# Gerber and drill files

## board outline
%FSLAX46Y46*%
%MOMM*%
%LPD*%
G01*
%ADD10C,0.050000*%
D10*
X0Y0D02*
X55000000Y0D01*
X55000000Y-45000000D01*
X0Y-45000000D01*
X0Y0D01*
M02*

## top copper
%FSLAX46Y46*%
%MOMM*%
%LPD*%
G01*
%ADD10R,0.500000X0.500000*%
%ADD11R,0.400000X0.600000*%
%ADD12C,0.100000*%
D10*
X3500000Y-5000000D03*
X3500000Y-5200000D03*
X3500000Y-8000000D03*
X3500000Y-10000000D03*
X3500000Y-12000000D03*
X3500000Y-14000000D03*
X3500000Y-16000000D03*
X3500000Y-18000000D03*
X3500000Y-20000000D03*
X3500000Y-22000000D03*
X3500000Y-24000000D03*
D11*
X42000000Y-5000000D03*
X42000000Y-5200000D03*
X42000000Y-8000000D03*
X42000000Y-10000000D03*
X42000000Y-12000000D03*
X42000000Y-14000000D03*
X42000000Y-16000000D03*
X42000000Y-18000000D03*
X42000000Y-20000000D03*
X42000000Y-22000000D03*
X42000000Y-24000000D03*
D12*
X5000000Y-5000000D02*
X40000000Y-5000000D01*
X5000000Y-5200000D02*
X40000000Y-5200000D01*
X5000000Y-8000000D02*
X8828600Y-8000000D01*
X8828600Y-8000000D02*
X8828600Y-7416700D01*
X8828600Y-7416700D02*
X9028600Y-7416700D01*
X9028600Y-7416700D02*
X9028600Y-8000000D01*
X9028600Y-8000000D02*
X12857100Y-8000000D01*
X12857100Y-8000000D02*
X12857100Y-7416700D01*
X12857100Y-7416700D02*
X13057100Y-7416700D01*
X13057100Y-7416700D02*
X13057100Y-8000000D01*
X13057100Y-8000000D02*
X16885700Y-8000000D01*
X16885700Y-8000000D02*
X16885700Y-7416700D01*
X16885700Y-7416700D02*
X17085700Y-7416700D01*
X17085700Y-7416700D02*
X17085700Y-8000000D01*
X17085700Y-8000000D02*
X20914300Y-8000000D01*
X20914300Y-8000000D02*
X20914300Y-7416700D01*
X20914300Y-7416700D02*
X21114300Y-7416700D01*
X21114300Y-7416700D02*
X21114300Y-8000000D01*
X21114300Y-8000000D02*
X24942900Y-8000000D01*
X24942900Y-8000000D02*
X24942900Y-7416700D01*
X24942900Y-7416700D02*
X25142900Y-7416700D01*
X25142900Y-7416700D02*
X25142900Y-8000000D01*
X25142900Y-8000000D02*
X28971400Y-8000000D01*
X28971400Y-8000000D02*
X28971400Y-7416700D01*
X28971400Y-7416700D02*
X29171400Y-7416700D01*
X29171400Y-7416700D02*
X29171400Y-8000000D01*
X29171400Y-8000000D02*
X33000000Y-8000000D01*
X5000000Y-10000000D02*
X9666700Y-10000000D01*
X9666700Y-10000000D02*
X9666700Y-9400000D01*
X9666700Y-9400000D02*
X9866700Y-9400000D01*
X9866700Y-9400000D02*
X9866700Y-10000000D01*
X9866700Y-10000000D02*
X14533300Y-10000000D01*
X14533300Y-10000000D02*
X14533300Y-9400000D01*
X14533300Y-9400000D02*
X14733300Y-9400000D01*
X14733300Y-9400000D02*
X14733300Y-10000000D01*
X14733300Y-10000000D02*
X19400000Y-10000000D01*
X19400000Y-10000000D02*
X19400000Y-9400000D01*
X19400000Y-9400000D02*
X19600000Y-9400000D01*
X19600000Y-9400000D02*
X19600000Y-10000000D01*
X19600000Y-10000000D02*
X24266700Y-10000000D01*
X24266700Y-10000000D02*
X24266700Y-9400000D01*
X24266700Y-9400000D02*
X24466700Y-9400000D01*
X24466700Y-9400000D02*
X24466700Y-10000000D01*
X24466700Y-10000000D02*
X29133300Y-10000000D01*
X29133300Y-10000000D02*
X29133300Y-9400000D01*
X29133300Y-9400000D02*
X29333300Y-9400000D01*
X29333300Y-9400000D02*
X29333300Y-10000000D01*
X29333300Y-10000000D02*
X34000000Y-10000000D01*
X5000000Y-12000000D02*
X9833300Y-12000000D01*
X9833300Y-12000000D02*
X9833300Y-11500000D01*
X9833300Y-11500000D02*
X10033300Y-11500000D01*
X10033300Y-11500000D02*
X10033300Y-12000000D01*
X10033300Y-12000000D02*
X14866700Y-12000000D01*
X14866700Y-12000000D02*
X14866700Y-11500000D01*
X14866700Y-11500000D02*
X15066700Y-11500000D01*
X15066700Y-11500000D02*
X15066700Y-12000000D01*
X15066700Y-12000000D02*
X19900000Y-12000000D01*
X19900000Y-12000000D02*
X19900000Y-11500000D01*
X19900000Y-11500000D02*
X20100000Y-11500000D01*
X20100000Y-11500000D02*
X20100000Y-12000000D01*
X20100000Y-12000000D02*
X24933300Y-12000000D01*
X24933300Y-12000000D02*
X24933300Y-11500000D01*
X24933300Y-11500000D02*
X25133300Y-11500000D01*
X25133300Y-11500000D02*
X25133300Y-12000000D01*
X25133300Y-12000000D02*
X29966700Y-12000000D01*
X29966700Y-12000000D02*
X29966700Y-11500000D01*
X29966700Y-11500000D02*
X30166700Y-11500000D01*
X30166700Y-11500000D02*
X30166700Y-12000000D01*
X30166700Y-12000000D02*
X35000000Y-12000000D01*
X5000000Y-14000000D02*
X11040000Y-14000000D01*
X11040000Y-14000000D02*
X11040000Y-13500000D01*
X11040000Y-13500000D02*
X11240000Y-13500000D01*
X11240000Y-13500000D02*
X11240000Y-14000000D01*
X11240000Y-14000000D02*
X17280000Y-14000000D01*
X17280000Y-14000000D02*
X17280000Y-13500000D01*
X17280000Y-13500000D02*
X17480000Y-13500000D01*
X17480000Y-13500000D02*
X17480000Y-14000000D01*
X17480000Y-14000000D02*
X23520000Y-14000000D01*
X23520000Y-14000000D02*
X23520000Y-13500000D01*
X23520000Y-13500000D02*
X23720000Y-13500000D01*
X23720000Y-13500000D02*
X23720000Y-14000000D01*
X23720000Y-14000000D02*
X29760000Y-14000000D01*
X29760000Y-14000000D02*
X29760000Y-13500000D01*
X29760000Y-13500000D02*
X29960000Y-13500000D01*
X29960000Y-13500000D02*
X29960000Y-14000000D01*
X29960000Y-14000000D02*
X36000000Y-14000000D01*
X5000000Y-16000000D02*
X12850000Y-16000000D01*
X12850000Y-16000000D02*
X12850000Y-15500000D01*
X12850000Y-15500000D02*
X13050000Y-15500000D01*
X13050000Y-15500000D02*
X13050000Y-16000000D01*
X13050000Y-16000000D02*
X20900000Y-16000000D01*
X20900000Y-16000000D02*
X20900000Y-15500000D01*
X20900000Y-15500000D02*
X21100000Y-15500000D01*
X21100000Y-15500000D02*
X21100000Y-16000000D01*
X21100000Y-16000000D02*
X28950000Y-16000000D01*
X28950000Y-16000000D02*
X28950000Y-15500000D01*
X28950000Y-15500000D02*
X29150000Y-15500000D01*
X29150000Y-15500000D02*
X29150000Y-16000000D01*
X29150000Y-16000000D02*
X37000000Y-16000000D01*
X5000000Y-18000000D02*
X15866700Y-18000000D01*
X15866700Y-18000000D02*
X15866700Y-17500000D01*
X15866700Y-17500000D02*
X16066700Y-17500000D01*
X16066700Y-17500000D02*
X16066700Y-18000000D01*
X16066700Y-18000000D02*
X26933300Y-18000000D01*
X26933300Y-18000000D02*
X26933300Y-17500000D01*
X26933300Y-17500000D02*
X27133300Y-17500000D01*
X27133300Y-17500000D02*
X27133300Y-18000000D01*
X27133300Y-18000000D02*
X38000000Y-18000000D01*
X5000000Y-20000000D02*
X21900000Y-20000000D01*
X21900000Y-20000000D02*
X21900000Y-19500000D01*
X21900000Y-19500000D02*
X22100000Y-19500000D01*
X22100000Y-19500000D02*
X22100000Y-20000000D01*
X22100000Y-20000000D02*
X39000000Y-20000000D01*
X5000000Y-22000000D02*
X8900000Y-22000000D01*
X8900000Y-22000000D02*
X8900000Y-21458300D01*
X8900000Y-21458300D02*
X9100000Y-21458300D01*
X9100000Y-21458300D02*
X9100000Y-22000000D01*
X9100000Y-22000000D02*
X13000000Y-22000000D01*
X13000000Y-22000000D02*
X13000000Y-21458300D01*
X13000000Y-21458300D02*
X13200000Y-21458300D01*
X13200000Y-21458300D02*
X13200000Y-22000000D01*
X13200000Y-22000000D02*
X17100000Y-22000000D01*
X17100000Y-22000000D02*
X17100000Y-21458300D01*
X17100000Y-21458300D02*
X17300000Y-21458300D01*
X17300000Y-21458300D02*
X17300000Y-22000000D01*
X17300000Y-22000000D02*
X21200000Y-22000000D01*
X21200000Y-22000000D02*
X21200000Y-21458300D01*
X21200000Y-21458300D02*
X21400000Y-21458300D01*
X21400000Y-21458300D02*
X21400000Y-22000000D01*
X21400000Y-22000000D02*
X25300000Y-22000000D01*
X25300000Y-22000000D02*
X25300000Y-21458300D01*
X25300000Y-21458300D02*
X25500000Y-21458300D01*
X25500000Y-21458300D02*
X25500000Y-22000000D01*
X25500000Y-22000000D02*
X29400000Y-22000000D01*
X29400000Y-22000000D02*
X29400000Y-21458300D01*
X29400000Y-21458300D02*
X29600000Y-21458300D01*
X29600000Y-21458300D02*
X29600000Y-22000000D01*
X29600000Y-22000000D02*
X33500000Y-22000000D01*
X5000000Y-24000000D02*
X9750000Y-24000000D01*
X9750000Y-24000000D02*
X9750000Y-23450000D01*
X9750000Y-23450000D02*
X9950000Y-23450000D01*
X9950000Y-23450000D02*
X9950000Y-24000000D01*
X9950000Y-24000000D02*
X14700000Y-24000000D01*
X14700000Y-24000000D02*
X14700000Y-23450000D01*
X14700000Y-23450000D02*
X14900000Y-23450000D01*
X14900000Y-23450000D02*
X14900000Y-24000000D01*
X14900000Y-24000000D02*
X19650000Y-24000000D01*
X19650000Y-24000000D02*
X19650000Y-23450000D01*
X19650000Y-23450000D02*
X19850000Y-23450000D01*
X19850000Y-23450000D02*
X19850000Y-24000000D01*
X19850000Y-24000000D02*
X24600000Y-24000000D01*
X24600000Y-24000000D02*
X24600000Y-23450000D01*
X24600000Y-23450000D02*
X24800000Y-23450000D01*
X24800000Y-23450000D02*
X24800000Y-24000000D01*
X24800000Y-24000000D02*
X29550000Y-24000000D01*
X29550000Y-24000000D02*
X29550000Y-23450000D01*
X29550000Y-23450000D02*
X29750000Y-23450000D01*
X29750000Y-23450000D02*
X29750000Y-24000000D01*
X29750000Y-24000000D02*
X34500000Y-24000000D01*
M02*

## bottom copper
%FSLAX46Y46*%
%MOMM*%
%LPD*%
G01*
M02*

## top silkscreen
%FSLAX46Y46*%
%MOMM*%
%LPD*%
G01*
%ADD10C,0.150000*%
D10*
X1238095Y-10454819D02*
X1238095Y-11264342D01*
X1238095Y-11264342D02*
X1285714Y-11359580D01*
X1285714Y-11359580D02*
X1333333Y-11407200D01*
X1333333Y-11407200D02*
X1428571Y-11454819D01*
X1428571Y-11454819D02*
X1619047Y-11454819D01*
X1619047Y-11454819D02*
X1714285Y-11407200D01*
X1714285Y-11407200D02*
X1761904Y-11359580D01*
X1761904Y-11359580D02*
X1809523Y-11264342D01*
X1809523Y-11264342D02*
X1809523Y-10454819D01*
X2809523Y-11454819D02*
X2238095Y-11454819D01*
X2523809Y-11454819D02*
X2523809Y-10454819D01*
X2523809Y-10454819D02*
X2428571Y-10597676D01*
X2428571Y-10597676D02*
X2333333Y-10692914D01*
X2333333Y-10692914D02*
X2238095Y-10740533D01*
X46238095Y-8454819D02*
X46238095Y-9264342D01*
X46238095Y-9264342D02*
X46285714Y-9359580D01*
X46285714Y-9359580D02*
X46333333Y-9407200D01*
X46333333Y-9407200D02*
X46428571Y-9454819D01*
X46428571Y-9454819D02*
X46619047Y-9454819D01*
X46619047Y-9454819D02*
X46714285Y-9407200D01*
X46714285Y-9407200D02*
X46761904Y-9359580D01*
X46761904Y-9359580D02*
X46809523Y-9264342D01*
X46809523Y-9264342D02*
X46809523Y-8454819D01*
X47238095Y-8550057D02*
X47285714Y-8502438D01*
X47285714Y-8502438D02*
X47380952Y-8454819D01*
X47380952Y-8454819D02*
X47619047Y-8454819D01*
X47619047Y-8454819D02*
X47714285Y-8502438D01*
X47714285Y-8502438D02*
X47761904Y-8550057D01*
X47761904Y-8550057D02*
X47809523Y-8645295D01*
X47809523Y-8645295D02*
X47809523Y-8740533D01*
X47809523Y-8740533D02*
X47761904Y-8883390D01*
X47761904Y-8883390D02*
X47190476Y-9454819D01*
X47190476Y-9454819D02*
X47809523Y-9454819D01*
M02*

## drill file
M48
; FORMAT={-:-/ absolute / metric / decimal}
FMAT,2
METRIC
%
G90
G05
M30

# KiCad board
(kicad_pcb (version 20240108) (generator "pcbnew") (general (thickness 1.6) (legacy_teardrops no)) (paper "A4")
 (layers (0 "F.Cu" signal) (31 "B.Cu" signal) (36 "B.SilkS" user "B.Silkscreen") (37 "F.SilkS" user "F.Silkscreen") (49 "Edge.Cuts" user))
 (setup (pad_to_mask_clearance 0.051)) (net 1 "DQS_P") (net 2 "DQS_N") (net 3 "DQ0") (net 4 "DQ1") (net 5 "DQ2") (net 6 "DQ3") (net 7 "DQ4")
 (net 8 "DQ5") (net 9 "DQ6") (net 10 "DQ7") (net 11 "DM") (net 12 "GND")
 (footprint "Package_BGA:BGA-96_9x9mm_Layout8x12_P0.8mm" (layer "F.Cu") (at 2 18)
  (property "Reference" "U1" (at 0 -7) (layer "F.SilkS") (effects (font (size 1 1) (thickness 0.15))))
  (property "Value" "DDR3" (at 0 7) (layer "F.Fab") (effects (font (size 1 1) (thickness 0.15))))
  (pad "A1" smd rect (at 1.5 -13) (size 0.5 0.5) (layers "F.Cu" "F.Paste" "F.Mask") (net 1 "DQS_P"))
  (pad "A2" smd rect (at 1.5 -12.8) (size 0.5 0.5) (layers "F.Cu" "F.Paste" "F.Mask") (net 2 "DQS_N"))
  (pad "B1" smd rect (at 1.5 -10) (size 0.5 0.5) (layers "F.Cu" "F.Paste" "F.Mask") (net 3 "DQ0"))
  (pad "B2" smd rect (at 1.5 -8) (size 0.5 0.5) (layers "F.Cu" "F.Paste" "F.Mask") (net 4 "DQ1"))
  (pad "B3" smd rect (at 1.5 -6) (size 0.5 0.5) (layers "F.Cu" "F.Paste" "F.Mask") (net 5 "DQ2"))
  (pad "B4" smd rect (at 1.5 -4) (size 0.5 0.5) (layers "F.Cu" "F.Paste" "F.Mask") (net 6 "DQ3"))
  (pad "B5" smd rect (at 1.5 -2) (size 0.5 0.5) (layers "F.Cu" "F.Paste" "F.Mask") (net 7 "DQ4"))
  (pad "B6" smd rect (at 1.5 0) (size 0.5 0.5) (layers "F.Cu" "F.Paste" "F.Mask") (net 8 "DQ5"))
  (pad "B7" smd rect (at 1.5 2) (size 0.5 0.5) (layers "F.Cu" "F.Paste" "F.Mask") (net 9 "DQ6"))
  (pad "B8" smd rect (at 1.5 4) (size 0.5 0.5) (layers "F.Cu" "F.Paste" "F.Mask") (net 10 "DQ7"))
  (pad "B9" smd rect (at 1.5 6) (size 0.5 0.5) (layers "F.Cu" "F.Paste" "F.Mask") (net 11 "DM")))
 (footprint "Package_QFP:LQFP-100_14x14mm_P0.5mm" (layer "F.Cu") (at 47 18)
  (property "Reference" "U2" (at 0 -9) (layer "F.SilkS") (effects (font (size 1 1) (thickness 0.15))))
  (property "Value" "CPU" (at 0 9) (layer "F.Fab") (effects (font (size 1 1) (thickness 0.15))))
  (pad "1" smd rect (at -5 -13) (size 0.4 0.6) (layers "F.Cu" "F.Paste" "F.Mask") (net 1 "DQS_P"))
  (pad "2" smd rect (at -5 -12.8) (size 0.4 0.6) (layers "F.Cu" "F.Paste" "F.Mask") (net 2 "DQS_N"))
  (pad "3" smd rect (at -5 -10) (size 0.4 0.6) (layers "F.Cu" "F.Paste" "F.Mask") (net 3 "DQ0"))
  (pad "4" smd rect (at -5 -8) (size 0.4 0.6) (layers "F.Cu" "F.Paste" "F.Mask") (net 4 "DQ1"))
  (pad "5" smd rect (at -5 -6) (size 0.4 0.6) (layers "F.Cu" "F.Paste" "F.Mask") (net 5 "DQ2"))
  (pad "6" smd rect (at -5 -4) (size 0.4 0.6) (layers "F.Cu" "F.Paste" "F.Mask") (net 6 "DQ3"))
  (pad "7" smd rect (at -5 -2) (size 0.4 0.6) (layers "F.Cu" "F.Paste" "F.Mask") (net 7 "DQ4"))
  (pad "8" smd rect (at -5 0) (size 0.4 0.6) (layers "F.Cu" "F.Paste" "F.Mask") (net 8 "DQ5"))
  (pad "9" smd rect (at -5 2) (size 0.4 0.6) (layers "F.Cu" "F.Paste" "F.Mask") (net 9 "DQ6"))
  (pad "10" smd rect (at -5 4) (size 0.4 0.6) (layers "F.Cu" "F.Paste" "F.Mask") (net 10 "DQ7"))
  (pad "11" smd rect (at -5 6) (size 0.4 0.6) (layers "F.Cu" "F.Paste" "F.Mask") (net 11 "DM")))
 (segment (start 5 5) (end 40 5) (width 0.1) (layer "F.Cu") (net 1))
 (segment (start 5 5.2) (end 40 5.2) (width 0.1) (layer "F.Cu") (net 2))
 (segment (start 5.0000 8.0) (end 8.8286 8.0) (width 0.1) (layer "F.Cu") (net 3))
 (segment (start 8.8286 8.0) (end 8.8286 7.4167) (width 0.1) (layer "F.Cu") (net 3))
 (segment (start 8.8286 7.4167) (end 9.0286 7.4167) (width 0.1) (layer "F.Cu") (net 3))
 (segment (start 9.0286 7.4167) (end 9.0286 8.0) (width 0.1) (layer "F.Cu") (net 3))
 (segment (start 9.0286 8.0) (end 12.8571 8.0) (width 0.1) (layer "F.Cu") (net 3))
 (segment (start 12.8571 8.0) (end 12.8571 7.4167) (width 0.1) (layer "F.Cu") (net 3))
 (segment (start 12.8571 7.4167) (end 13.0571 7.4167) (width 0.1) (layer "F.Cu") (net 3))
 (segment (start 13.0571 7.4167) (end 13.0571 8.0) (width 0.1) (layer "F.Cu") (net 3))
 (segment (start 13.0571 8.0) (end 16.8857 8.0) (width 0.1) (layer "F.Cu") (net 3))
 (segment (start 16.8857 8.0) (end 16.8857 7.4167) (width 0.1) (layer "F.Cu") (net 3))
 (segment (start 16.8857 7.4167) (end 17.0857 7.4167) (width 0.1) (layer "F.Cu") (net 3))
 (segment (start 17.0857 7.4167) (end 17.0857 8.0) (width 0.1) (layer "F.Cu") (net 3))
 (segment (start 17.0857 8.0) (end 20.9143 8.0) (width 0.1) (layer "F.Cu") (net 3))
 (segment (start 20.9143 8.0) (end 20.9143 7.4167) (width 0.1) (layer "F.Cu") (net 3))
 (segment (start 20.9143 7.4167) (end 21.1143 7.4167) (width 0.1) (layer "F.Cu") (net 3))
 (segment (start 21.1143 7.4167) (end 21.1143 8.0) (width 0.1) (layer "F.Cu") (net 3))
 (segment (start 21.1143 8.0) (end 24.9429 8.0) (width 0.1) (layer "F.Cu") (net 3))
 (segment (start 24.9429 8.0) (end 24.9429 7.4167) (width 0.1) (layer "F.Cu") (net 3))
 (segment (start 24.9429 7.4167) (end 25.1429 7.4167) (width 0.1) (layer "F.Cu") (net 3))
 (segment (start 25.1429 7.4167) (end 25.1429 8.0) (width 0.1) (layer "F.Cu") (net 3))
 (segment (start 25.1429 8.0) (end 28.9714 8.0) (width 0.1) (layer "F.Cu") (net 3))
 (segment (start 28.9714 8.0) (end 28.9714 7.4167) (width 0.1) (layer "F.Cu") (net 3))
 (segment (start 28.9714 7.4167) (end 29.1714 7.4167) (width 0.1) (layer "F.Cu") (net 3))
 (segment (start 29.1714 7.4167) (end 29.1714 8.0) (width 0.1) (layer "F.Cu") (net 3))
 (segment (start 29.1714 8.0) (end 33.0 8.0) (width 0.1) (layer "F.Cu") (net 3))
 (segment (start 5.0000 10.0) (end 9.6667 10.0) (width 0.1) (layer "F.Cu") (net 4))
 (segment (start 9.6667 10.0) (end 9.6667 9.4000) (width 0.1) (layer "F.Cu") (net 4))
 (segment (start 9.6667 9.4000) (end 9.8667 9.4000) (width 0.1) (layer "F.Cu") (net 4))
 (segment (start 9.8667 9.4000) (end 9.8667 10.0) (width 0.1) (layer "F.Cu") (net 4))
 (segment (start 9.8667 10.0) (end 14.5333 10.0) (width 0.1) (layer "F.Cu") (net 4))
 (segment (start 14.5333 10.0) (end 14.5333 9.4000) (width 0.1) (layer "F.Cu") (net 4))
 (segment (start 14.5333 9.4000) (end 14.7333 9.4000) (width 0.1) (layer "F.Cu") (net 4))
 (segment (start 14.7333 9.4000) (end 14.7333 10.0) (width 0.1) (layer "F.Cu") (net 4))
 (segment (start 14.7333 10.0) (end 19.4000 10.0) (width 0.1) (layer "F.Cu") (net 4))
 (segment (start 19.4000 10.0) (end 19.4000 9.4000) (width 0.1) (layer "F.Cu") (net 4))
 (segment (start 19.4000 9.4000) (end 19.6000 9.4000) (width 0.1) (layer "F.Cu") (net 4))
 (segment (start 19.6000 9.4000) (end 19.6000 10.0) (width 0.1) (layer "F.Cu") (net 4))
 (segment (start 19.6000 10.0) (end 24.2667 10.0) (width 0.1) (layer "F.Cu") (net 4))
 (segment (start 24.2667 10.0) (end 24.2667 9.4000) (width 0.1) (layer "F.Cu") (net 4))
 (segment (start 24.2667 9.4000) (end 24.4667 9.4000) (width 0.1) (layer "F.Cu") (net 4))
 (segment (start 24.4667 9.4000) (end 24.4667 10.0) (width 0.1) (layer "F.Cu") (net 4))
 (segment (start 24.4667 10.0) (end 29.1333 10.0) (width 0.1) (layer "F.Cu") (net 4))
 (segment (start 29.1333 10.0) (end 29.1333 9.4000) (width 0.1) (layer "F.Cu") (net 4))
 (segment (start 29.1333 9.4000) (end 29.3333 9.4000) (width 0.1) (layer "F.Cu") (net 4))
 (segment (start 29.3333 9.4000) (end 29.3333 10.0) (width 0.1) (layer "F.Cu") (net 4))
 (segment (start 29.3333 10.0) (end 34.0 10.0) (width 0.1) (layer "F.Cu") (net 4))
 (segment (start 5.0000 12.0) (end 9.8333 12.0) (width 0.1) (layer "F.Cu") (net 5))
 (segment (start 9.8333 12.0) (end 9.8333 11.5000) (width 0.1) (layer "F.Cu") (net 5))
 (segment (start 9.8333 11.5000) (end 10.0333 11.5000) (width 0.1) (layer "F.Cu") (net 5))
 (segment (start 10.0333 11.5000) (end 10.0333 12.0) (width 0.1) (layer "F.Cu") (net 5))
 (segment (start 10.0333 12.0) (end 14.8667 12.0) (width 0.1) (layer "F.Cu") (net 5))
 (segment (start 14.8667 12.0) (end 14.8667 11.5000) (width 0.1) (layer "F.Cu") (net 5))
 (segment (start 14.8667 11.5000) (end 15.0667 11.5000) (width 0.1) (layer "F.Cu") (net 5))
 (segment (start 15.0667 11.5000) (end 15.0667 12.0) (width 0.1) (layer "F.Cu") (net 5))
 (segment (start 15.0667 12.0) (end 19.9000 12.0) (width 0.1) (layer "F.Cu") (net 5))
 (segment (start 19.9000 12.0) (end 19.9000 11.5000) (width 0.1) (layer "F.Cu") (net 5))
 (segment (start 19.9000 11.5000) (end 20.1000 11.5000) (width 0.1) (layer "F.Cu") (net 5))
 (segment (start 20.1000 11.5000) (end 20.1000 12.0) (width 0.1) (layer "F.Cu") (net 5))
 (segment (start 20.1000 12.0) (end 24.9333 12.0) (width 0.1) (layer "F.Cu") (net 5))
 (segment (start 24.9333 12.0) (end 24.9333 11.5000) (width 0.1) (layer "F.Cu") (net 5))
 (segment (start 24.9333 11.5000) (end 25.1333 11.5000) (width 0.1) (layer "F.Cu") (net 5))
 (segment (start 25.1333 11.5000) (end 25.1333 12.0) (width 0.1) (layer "F.Cu") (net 5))
 (segment (start 25.1333 12.0) (end 29.9667 12.0) (width 0.1) (layer "F.Cu") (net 5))
 (segment (start 29.9667 12.0) (end 29.9667 11.5000) (width 0.1) (layer "F.Cu") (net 5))
 (segment (start 29.9667 11.5000) (end 30.1667 11.5000) (width 0.1) (layer "F.Cu") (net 5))
 (segment (start 30.1667 11.5000) (end 30.1667 12.0) (width 0.1) (layer "F.Cu") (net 5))
 (segment (start 30.1667 12.0) (end 35.0 12.0) (width 0.1) (layer "F.Cu") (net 5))
 (segment (start 5.0000 14.0) (end 11.0400 14.0) (width 0.1) (layer "F.Cu") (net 6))
 (segment (start 11.0400 14.0) (end 11.0400 13.5000) (width 0.1) (layer "F.Cu") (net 6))
 (segment (start 11.0400 13.5000) (end 11.2400 13.5000) (width 0.1) (layer "F.Cu") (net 6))
 (segment (start 11.2400 13.5000) (end 11.2400 14.0) (width 0.1) (layer "F.Cu") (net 6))
 (segment (start 11.2400 14.0) (end 17.2800 14.0) (width 0.1) (layer "F.Cu") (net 6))
 (segment (start 17.2800 14.0) (end 17.2800 13.5000) (width 0.1) (layer "F.Cu") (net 6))
 (segment (start 17.2800 13.5000) (end 17.4800 13.5000) (width 0.1) (layer "F.Cu") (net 6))
 (segment (start 17.4800 13.5000) (end 17.4800 14.0) (width 0.1) (layer "F.Cu") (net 6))
 (segment (start 17.4800 14.0) (end 23.5200 14.0) (width 0.1) (layer "F.Cu") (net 6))
 (segment (start 23.5200 14.0) (end 23.5200 13.5000) (width 0.1) (layer "F.Cu") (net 6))
 (segment (start 23.5200 13.5000) (end 23.7200 13.5000) (width 0.1) (layer "F.Cu") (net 6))
 (segment (start 23.7200 13.5000) (end 23.7200 14.0) (width 0.1) (layer "F.Cu") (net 6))
 (segment (start 23.7200 14.0) (end 29.7600 14.0) (width 0.1) (layer "F.Cu") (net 6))
 (segment (start 29.7600 14.0) (end 29.7600 13.5000) (width 0.1) (layer "F.Cu") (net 6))
 (segment (start 29.7600 13.5000) (end 29.9600 13.5000) (width 0.1) (layer "F.Cu") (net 6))
 (segment (start 29.9600 13.5000) (end 29.9600 14.0) (width 0.1) (layer "F.Cu") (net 6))
 (segment (start 29.9600 14.0) (end 36.0 14.0) (width 0.1) (layer "F.Cu") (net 6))
 (segment (start 5.0000 16.0) (end 12.8500 16.0) (width 0.1) (layer "F.Cu") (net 7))
 (segment (start 12.8500 16.0) (end 12.8500 15.5000) (width 0.1) (layer "F.Cu") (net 7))
 (segment (start 12.8500 15.5000) (end 13.0500 15.5000) (width 0.1) (layer "F.Cu") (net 7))
 (segment (start 13.0500 15.5000) (end 13.0500 16.0) (width 0.1) (layer "F.Cu") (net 7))
 (segment (start 13.0500 16.0) (end 20.9000 16.0) (width 0.1) (layer "F.Cu") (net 7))
 (segment (start 20.9000 16.0) (end 20.9000 15.5000) (width 0.1) (layer "F.Cu") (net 7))
 (segment (start 20.9000 15.5000) (end 21.1000 15.5000) (width 0.1) (layer "F.Cu") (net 7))
 (segment (start 21.1000 15.5000) (end 21.1000 16.0) (width 0.1) (layer "F.Cu") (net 7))
 (segment (start 21.1000 16.0) (end 28.9500 16.0) (width 0.1) (layer "F.Cu") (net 7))
 (segment (start 28.9500 16.0) (end 28.9500 15.5000) (width 0.1) (layer "F.Cu") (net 7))
 (segment (start 28.9500 15.5000) (end 29.1500 15.5000) (width 0.1) (layer "F.Cu") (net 7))
 (segment (start 29.1500 15.5000) (end 29.1500 16.0) (width 0.1) (layer "F.Cu") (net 7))
 (segment (start 29.1500 16.0) (end 37.0 16.0) (width 0.1) (layer "F.Cu") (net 7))
 (segment (start 5.0000 18.0) (end 15.8667 18.0) (width 0.1) (layer "F.Cu") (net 8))
 (segment (start 15.8667 18.0) (end 15.8667 17.5000) (width 0.1) (layer "F.Cu") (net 8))
 (segment (start 15.8667 17.5000) (end 16.0667 17.5000) (width 0.1) (layer "F.Cu") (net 8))
 (segment (start 16.0667 17.5000) (end 16.0667 18.0) (width 0.1) (layer "F.Cu") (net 8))
 (segment (start 16.0667 18.0) (end 26.9333 18.0) (width 0.1) (layer "F.Cu") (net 8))
 (segment (start 26.9333 18.0) (end 26.9333 17.5000) (width 0.1) (layer "F.Cu") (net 8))
 (segment (start 26.9333 17.5000) (end 27.1333 17.5000) (width 0.1) (layer "F.Cu") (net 8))
 (segment (start 27.1333 17.5000) (end 27.1333 18.0) (width 0.1) (layer "F.Cu") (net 8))
 (segment (start 27.1333 18.0) (end 38.0 18.0) (width 0.1) (layer "F.Cu") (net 8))
 (segment (start 5.0000 20.0) (end 21.9000 20.0) (width 0.1) (layer "F.Cu") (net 9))
 (segment (start 21.9000 20.0) (end 21.9000 19.5000) (width 0.1) (layer "F.Cu") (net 9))
 (segment (start 21.9000 19.5000) (end 22.1000 19.5000) (width 0.1) (layer "F.Cu") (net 9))
 (segment (start 22.1000 19.5000) (end 22.1000 20.0) (width 0.1) (layer "F.Cu") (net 9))
 (segment (start 22.1000 20.0) (end 39.0 20.0) (width 0.1) (layer "F.Cu") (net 9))
 (segment (start 5.0000 22.0) (end 8.9000 22.0) (width 0.1) (layer "F.Cu") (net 10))
 (segment (start 8.9000 22.0) (end 8.9000 21.4583) (width 0.1) (layer "F.Cu") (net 10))
 (segment (start 8.9000 21.4583) (end 9.1000 21.4583) (width 0.1) (layer "F.Cu") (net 10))
 (segment (start 9.1000 21.4583) (end 9.1000 22.0) (width 0.1) (layer "F.Cu") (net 10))
 (segment (start 9.1000 22.0) (end 13.0000 22.0) (width 0.1) (layer "F.Cu") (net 10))
 (segment (start 13.0000 22.0) (end 13.0000 21.4583) (width 0.1) (layer "F.Cu") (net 10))
 (segment (start 13.0000 21.4583) (end 13.2000 21.4583) (width 0.1) (layer "F.Cu") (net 10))
 (segment (start 13.2000 21.4583) (end 13.2000 22.0) (width 0.1) (layer "F.Cu") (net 10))
 (segment (start 13.2000 22.0) (end 17.1000 22.0) (width 0.1) (layer "F.Cu") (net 10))
 (segment (start 17.1000 22.0) (end 17.1000 21.4583) (width 0.1) (layer "F.Cu") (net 10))
 (segment (start 17.1000 21.4583) (end 17.3000 21.4583) (width 0.1) (layer "F.Cu") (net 10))
 (segment (start 17.3000 21.4583) (end 17.3000 22.0) (width 0.1) (layer "F.Cu") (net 10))
 (segment (start 17.3000 22.0) (end 21.2000 22.0) (width 0.1) (layer "F.Cu") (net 10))
 (segment (start 21.2000 22.0) (end 21.2000 21.4583) (width 0.1) (layer "F.Cu") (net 10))
 (segment (start 21.2000 21.4583) (end 21.4000 21.4583) (width 0.1) (layer "F.Cu") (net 10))
 (segment (start 21.4000 21.4583) (end 21.4000 22.0) (width 0.1) (layer "F.Cu") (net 10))
 (segment (start 21.4000 22.0) (end 25.3000 22.0) (width 0.1) (layer "F.Cu") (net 10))
 (segment (start 25.3000 22.0) (end 25.3000 21.4583) (width 0.1) (layer "F.Cu") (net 10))
 (segment (start 25.3000 21.4583) (end 25.5000 21.4583) (width 0.1) (layer "F.Cu") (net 10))
 (segment (start 25.5000 21.4583) (end 25.5000 22.0) (width 0.1) (layer "F.Cu") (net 10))
 (segment (start 25.5000 22.0) (end 29.4000 22.0) (width 0.1) (layer "F.Cu") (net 10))
 (segment (start 29.4000 22.0) (end 29.4000 21.4583) (width 0.1) (layer "F.Cu") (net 10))
 (segment (start 29.4000 21.4583) (end 29.6000 21.4583) (width 0.1) (layer "F.Cu") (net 10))
 (segment (start 29.6000 21.4583) (end 29.6000 22.0) (width 0.1) (layer "F.Cu") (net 10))
 (segment (start 29.6000 22.0) (end 33.5 22.0) (width 0.1) (layer "F.Cu") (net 10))
 (segment (start 5.0000 24.0) (end 9.7500 24.0) (width 0.1) (layer "F.Cu") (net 11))
 (segment (start 9.7500 24.0) (end 9.7500 23.4500) (width 0.1) (layer "F.Cu") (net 11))
 (segment (start 9.7500 23.4500) (end 9.9500 23.4500) (width 0.1) (layer "F.Cu") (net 11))
 (segment (start 9.9500 23.4500) (end 9.9500 24.0) (width 0.1) (layer "F.Cu") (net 11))
 (segment (start 9.9500 24.0) (end 14.7000 24.0) (width 0.1) (layer "F.Cu") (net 11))
 (segment (start 14.7000 24.0) (end 14.7000 23.4500) (width 0.1) (layer "F.Cu") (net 11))
 (segment (start 14.7000 23.4500) (end 14.9000 23.4500) (width 0.1) (layer "F.Cu") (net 11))
 (segment (start 14.9000 23.4500) (end 14.9000 24.0) (width 0.1) (layer "F.Cu") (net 11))
 (segment (start 14.9000 24.0) (end 19.6500 24.0) (width 0.1) (layer "F.Cu") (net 11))
 (segment (start 19.6500 24.0) (end 19.6500 23.4500) (width 0.1) (layer "F.Cu") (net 11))
 (segment (start 19.6500 23.4500) (end 19.8500 23.4500) (width 0.1) (layer "F.Cu") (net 11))
 (segment (start 19.8500 23.4500) (end 19.8500 24.0) (width 0.1) (layer "F.Cu") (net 11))
 (segment (start 19.8500 24.0) (end 24.6000 24.0) (width 0.1) (layer "F.Cu") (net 11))
 (segment (start 24.6000 24.0) (end 24.6000 23.4500) (width 0.1) (layer "F.Cu") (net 11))
 (segment (start 24.6000 23.4500) (end 24.8000 23.4500) (width 0.1) (layer "F.Cu") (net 11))
 (segment (start 24.8000 23.4500) (end 24.8000 24.0) (width 0.1) (layer "F.Cu") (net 11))
 (segment (start 24.8000 24.0) (end 29.5500 24.0) (width 0.1) (layer "F.Cu") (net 11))
 (segment (start 29.5500 24.0) (end 29.5500 23.4500) (width 0.1) (layer "F.Cu") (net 11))
 (segment (start 29.5500 23.4500) (end 29.7500 23.4500) (width 0.1) (layer "F.Cu") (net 11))
 (segment (start 29.7500 23.4500) (end 29.7500 24.0) (width 0.1) (layer "F.Cu") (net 11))
 (segment (start 29.7500 24.0) (end 34.5 24.0) (width 0.1) (layer "F.Cu") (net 11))
 (gr_rect (start 0 0) (end 55 45) (layer "Edge.Cuts") (width 0.05)))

